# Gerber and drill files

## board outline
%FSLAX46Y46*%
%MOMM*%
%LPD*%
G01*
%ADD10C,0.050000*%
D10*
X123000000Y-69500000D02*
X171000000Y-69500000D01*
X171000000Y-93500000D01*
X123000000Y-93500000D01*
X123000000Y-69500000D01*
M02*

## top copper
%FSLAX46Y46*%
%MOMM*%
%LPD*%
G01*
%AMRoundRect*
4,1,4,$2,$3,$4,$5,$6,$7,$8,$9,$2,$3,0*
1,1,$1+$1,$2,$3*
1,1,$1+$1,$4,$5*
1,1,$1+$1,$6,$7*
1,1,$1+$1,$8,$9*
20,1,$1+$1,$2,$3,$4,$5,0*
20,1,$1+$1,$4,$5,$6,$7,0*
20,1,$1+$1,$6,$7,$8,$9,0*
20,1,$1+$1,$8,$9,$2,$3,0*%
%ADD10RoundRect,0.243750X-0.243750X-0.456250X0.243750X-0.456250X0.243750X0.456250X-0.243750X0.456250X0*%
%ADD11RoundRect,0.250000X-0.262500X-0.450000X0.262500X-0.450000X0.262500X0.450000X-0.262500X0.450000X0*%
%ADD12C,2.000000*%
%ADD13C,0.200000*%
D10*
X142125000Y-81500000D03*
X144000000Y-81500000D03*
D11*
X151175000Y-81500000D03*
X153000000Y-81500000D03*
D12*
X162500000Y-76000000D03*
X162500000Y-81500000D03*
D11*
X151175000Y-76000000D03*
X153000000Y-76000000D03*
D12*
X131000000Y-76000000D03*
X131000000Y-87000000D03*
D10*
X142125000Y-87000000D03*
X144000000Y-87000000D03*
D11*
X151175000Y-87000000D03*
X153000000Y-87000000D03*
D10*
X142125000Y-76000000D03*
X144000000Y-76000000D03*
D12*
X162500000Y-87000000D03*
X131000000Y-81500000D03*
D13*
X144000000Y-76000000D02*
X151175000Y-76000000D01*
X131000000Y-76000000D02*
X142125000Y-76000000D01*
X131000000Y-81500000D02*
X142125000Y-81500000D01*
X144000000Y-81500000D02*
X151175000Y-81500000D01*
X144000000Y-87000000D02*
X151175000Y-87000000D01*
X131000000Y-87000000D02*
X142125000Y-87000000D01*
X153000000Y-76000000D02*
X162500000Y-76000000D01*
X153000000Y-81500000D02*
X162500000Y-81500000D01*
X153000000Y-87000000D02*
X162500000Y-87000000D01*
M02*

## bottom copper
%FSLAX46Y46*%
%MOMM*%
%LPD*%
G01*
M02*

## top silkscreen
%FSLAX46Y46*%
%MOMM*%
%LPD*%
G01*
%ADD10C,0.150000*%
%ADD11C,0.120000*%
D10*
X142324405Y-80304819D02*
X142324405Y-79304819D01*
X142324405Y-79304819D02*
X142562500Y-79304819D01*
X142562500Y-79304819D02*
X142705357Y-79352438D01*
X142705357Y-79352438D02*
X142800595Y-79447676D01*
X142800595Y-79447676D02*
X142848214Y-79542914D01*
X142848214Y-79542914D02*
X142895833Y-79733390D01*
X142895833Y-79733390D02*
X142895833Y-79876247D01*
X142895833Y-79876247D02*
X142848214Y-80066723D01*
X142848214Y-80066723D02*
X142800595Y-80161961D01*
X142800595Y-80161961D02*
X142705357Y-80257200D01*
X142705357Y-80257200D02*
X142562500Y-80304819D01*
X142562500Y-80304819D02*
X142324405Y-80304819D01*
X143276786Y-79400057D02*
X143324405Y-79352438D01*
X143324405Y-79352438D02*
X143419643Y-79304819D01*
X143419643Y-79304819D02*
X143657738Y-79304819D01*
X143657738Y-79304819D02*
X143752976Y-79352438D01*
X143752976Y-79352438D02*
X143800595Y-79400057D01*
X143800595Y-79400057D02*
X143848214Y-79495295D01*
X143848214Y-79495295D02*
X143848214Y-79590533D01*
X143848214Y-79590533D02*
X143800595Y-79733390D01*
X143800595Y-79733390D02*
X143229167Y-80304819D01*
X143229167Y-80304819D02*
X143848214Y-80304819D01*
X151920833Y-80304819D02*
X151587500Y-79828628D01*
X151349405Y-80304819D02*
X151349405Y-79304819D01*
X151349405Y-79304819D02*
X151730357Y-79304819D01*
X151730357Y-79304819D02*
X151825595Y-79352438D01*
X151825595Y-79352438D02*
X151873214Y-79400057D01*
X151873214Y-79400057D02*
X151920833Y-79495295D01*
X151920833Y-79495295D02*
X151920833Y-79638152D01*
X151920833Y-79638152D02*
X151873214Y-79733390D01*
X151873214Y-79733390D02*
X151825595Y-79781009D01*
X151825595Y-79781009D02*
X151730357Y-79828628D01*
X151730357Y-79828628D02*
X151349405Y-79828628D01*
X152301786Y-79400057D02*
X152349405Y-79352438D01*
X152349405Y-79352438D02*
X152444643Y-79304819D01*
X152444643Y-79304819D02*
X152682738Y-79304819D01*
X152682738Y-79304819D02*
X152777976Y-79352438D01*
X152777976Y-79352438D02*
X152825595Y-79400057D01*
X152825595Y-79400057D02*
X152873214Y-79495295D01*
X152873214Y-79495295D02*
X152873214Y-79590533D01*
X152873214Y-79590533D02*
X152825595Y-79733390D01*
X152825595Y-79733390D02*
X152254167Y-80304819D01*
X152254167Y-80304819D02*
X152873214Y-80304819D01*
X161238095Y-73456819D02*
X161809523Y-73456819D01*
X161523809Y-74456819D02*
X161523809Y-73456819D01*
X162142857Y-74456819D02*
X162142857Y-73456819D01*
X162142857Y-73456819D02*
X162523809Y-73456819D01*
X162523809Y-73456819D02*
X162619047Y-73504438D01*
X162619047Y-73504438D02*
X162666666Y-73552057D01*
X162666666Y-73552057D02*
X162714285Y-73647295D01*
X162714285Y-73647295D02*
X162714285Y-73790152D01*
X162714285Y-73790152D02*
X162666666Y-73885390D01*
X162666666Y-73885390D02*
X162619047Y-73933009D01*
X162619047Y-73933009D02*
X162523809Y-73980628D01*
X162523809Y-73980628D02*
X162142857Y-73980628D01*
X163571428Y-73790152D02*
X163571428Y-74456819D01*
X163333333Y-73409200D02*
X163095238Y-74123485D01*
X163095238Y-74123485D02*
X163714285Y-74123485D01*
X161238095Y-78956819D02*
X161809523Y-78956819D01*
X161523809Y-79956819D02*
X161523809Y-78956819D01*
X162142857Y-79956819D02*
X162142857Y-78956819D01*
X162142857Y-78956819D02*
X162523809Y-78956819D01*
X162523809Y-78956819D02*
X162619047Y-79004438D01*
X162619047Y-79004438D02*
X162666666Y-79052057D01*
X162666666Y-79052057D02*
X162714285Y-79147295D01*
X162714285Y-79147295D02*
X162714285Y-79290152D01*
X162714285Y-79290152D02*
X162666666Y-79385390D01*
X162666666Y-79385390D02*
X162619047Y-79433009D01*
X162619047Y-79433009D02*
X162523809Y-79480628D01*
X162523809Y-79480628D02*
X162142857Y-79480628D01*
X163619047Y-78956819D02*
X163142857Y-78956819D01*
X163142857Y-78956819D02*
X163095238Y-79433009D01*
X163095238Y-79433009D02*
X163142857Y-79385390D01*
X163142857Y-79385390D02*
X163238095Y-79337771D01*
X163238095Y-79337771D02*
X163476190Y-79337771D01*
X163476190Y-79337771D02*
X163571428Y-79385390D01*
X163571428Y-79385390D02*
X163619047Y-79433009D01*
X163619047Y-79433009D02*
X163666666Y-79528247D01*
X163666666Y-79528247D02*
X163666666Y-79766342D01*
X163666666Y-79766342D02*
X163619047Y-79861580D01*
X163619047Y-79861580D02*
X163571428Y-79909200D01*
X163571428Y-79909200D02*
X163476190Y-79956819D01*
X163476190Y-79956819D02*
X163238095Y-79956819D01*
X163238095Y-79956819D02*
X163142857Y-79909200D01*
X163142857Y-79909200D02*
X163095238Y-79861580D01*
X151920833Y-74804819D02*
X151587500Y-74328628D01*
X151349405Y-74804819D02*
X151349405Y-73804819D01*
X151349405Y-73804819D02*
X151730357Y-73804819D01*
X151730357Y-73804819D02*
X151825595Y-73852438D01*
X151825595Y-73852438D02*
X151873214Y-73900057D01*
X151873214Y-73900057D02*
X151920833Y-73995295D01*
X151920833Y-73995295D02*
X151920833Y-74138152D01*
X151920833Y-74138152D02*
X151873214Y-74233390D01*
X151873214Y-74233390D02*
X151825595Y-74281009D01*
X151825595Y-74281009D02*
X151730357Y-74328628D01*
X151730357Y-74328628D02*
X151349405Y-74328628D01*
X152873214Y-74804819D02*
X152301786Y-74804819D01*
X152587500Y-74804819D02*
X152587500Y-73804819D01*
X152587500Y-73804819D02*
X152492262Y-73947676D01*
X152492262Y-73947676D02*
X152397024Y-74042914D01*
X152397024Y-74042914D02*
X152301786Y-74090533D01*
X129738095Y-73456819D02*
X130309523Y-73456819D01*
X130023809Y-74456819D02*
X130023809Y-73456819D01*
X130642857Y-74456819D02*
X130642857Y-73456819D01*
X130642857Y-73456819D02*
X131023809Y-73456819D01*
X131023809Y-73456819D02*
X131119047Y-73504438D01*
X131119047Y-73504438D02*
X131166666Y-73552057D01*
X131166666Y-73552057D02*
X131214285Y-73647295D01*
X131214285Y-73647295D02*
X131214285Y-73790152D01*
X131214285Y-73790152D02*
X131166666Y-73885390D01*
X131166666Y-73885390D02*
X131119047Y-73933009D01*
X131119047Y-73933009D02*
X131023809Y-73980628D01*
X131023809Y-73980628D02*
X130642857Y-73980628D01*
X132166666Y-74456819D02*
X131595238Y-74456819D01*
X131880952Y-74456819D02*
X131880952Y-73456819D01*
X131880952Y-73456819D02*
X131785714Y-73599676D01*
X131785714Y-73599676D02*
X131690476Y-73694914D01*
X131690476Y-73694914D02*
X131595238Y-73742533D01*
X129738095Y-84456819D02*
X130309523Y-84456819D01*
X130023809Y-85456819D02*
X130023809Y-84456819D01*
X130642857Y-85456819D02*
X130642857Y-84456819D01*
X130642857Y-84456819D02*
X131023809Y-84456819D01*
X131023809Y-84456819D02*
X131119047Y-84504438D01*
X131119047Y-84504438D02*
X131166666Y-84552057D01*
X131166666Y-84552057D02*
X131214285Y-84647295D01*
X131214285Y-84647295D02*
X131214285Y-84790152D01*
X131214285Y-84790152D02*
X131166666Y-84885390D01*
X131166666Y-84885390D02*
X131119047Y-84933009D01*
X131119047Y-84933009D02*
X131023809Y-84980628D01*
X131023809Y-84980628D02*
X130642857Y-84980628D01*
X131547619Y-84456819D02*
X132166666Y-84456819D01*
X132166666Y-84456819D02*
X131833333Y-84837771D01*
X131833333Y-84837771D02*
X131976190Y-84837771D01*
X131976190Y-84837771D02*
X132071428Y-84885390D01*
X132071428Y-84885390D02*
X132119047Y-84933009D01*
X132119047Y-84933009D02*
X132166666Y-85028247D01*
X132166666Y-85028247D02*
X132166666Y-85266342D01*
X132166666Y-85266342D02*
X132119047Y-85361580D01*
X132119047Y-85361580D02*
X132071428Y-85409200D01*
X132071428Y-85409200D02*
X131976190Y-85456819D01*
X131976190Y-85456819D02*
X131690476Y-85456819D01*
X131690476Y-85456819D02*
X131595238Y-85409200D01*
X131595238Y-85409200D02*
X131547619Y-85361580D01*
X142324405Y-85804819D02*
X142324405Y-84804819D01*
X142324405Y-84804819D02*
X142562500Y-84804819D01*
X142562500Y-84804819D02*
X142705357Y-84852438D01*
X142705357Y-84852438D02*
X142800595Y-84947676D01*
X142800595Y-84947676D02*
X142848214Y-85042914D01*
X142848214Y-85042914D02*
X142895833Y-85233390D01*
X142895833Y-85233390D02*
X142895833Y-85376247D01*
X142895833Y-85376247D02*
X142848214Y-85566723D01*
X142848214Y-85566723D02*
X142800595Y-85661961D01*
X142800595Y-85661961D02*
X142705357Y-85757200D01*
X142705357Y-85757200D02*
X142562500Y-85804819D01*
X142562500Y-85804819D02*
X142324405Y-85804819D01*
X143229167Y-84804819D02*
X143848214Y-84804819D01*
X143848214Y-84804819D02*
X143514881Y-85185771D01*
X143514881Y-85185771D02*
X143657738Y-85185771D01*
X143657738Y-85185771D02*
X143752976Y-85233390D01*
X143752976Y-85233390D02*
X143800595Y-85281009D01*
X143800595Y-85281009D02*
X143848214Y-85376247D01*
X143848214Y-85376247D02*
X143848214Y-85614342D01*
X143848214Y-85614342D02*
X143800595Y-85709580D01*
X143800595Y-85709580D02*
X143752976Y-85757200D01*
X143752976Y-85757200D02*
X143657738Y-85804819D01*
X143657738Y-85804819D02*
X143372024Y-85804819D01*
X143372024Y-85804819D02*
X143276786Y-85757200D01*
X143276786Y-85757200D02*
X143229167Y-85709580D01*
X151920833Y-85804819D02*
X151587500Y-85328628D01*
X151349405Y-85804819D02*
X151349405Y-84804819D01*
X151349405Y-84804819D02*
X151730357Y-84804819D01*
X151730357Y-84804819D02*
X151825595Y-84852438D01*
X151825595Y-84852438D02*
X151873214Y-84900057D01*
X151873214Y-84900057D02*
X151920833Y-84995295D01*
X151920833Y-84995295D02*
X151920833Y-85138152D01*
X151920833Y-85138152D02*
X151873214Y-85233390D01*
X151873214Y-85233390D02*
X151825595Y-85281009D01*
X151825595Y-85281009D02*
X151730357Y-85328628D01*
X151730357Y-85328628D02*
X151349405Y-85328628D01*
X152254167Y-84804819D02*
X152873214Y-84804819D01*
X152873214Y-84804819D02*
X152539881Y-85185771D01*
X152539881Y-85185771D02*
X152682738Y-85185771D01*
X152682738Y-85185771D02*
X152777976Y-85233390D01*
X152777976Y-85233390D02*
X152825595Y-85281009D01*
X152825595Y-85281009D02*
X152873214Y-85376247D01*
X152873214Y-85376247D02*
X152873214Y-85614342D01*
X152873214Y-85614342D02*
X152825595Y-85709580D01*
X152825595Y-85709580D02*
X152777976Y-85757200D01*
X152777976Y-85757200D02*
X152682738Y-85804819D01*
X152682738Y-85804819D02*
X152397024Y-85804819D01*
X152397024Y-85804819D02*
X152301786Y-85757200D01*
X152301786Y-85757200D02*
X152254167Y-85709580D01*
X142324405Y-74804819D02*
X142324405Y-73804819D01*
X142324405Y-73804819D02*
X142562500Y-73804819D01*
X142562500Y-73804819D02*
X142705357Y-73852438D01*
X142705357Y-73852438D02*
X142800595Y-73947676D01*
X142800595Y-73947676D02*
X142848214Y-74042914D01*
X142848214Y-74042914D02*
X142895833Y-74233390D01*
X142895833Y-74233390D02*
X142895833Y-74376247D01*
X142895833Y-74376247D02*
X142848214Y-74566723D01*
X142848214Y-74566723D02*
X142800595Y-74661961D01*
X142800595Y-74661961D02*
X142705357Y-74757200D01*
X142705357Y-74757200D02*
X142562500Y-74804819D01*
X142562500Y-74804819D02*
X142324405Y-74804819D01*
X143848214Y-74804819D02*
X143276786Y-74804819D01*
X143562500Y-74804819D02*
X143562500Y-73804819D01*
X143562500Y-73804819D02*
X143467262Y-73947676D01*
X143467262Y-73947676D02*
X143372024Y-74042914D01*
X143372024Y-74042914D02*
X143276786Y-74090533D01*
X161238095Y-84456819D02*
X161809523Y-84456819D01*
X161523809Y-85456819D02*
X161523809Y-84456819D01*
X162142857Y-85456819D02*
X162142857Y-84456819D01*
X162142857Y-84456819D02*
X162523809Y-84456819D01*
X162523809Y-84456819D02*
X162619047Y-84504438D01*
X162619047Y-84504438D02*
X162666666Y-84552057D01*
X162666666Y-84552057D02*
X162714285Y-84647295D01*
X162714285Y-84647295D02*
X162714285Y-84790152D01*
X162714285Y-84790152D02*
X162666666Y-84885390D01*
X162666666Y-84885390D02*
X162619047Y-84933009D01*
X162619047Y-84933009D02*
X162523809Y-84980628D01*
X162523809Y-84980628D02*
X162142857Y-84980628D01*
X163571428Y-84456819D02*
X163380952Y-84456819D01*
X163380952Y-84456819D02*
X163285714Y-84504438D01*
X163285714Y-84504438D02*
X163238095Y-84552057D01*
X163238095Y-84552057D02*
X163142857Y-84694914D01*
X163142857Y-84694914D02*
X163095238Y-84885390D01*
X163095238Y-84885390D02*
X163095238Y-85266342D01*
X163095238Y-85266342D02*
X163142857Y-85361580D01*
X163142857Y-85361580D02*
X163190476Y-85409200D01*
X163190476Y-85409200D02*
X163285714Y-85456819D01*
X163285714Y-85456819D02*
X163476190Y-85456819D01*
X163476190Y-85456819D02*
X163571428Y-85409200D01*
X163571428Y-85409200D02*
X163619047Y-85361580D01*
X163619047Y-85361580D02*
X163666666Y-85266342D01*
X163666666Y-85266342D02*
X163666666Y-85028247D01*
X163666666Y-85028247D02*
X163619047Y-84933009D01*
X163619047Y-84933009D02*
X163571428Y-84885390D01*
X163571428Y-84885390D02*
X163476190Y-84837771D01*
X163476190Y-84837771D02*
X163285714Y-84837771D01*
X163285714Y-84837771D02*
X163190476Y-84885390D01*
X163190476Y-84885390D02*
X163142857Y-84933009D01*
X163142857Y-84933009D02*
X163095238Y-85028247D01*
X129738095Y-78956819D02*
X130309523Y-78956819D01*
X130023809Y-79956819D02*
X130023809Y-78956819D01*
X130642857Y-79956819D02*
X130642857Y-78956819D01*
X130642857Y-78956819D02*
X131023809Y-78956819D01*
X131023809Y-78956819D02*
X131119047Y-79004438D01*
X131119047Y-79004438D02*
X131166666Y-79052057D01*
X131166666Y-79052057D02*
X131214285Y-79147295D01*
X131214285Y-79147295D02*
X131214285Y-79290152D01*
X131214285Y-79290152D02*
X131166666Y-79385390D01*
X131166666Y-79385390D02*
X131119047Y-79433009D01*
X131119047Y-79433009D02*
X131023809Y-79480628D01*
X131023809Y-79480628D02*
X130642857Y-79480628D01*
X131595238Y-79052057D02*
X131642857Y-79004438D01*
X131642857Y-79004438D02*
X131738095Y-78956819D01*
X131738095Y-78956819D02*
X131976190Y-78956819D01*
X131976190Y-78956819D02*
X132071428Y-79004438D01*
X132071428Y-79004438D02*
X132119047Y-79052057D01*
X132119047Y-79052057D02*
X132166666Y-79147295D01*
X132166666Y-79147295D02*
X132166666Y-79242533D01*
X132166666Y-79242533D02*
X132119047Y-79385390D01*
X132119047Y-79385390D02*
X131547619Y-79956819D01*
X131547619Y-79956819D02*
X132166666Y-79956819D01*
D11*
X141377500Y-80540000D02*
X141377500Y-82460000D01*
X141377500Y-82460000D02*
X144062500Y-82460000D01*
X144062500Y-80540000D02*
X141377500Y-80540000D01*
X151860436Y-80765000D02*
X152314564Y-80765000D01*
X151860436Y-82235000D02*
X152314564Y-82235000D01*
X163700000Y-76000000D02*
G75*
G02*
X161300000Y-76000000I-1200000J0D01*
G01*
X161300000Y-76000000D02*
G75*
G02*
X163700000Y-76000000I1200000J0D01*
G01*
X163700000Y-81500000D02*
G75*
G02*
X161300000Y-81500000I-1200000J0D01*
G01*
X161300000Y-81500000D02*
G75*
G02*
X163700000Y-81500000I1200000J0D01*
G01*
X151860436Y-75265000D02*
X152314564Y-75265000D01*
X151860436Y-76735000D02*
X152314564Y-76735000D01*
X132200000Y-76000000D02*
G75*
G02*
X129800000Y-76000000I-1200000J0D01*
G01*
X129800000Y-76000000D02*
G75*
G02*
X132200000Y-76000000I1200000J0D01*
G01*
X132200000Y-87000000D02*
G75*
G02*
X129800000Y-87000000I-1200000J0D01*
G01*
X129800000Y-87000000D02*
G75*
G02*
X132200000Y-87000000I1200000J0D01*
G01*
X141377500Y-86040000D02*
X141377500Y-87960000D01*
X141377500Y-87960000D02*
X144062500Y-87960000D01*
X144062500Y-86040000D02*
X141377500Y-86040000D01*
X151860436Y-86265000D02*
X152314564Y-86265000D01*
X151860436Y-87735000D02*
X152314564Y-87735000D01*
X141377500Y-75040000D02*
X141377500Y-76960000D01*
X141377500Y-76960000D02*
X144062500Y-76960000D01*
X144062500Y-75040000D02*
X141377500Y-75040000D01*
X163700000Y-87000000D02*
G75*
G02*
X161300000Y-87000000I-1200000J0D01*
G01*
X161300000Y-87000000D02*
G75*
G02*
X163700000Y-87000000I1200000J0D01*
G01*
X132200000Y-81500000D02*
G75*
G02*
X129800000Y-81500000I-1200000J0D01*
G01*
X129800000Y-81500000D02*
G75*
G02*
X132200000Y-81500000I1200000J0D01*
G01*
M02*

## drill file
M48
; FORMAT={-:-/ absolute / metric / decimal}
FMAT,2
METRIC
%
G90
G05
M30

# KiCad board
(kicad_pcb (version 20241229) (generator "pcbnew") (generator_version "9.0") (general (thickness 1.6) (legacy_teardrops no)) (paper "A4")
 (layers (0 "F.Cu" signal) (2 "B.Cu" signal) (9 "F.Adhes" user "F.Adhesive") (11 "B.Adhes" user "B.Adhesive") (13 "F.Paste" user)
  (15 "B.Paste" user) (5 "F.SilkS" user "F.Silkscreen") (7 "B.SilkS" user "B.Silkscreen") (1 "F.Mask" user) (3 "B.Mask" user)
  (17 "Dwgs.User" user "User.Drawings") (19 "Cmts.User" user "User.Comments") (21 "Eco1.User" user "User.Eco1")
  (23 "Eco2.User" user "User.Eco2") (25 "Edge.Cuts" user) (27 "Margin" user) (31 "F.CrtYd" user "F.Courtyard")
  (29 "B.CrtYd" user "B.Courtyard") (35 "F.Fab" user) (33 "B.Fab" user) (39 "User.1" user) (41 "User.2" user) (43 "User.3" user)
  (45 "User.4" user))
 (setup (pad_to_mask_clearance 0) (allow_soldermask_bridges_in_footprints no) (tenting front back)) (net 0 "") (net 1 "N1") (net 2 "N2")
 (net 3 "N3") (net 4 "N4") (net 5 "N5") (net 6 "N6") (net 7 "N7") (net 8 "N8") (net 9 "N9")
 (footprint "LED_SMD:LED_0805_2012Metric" (layer "F.Cu") (at 143.0625 81.5)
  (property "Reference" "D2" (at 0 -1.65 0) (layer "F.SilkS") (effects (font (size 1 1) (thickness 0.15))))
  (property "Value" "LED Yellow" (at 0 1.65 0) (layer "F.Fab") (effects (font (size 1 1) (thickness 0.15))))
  (fp_line (start -1.685 -0.96) (end -1.685 0.96) (stroke (width 0.12) (type solid)) (layer "F.SilkS"))
  (fp_line (start -1.685 0.96) (end 1 0.96) (stroke (width 0.12) (type solid)) (layer "F.SilkS"))
  (fp_line (start 1 -0.96) (end -1.685 -0.96) (stroke (width 0.12) (type solid)) (layer "F.SilkS"))
  (pad "1" smd roundrect (at -0.9375 0) (size 0.975 1.4) (layers "F.Cu" "F.Mask" "F.Paste") (roundrect_rratio 0.25) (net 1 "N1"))
  (pad "2" smd roundrect (at 0.9375 0) (size 0.975 1.4) (layers "F.Cu" "F.Mask" "F.Paste") (roundrect_rratio 0.25) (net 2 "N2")))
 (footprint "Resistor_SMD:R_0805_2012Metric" (layer "F.Cu") (at 152.0875 81.5)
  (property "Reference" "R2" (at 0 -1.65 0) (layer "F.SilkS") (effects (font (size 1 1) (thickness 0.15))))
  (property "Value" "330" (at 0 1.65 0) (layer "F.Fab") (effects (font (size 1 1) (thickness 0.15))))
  (fp_line (start -0.227064 -0.735) (end 0.227064 -0.735) (stroke (width 0.12) (type solid)) (layer "F.SilkS"))
  (fp_line (start -0.227064 0.735) (end 0.227064 0.735) (stroke (width 0.12) (type solid)) (layer "F.SilkS"))
  (pad "1" smd roundrect (at -0.9125 0) (size 1.025 1.4) (layers "F.Cu" "F.Mask" "F.Paste") (roundrect_rratio 0.243902) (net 2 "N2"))
  (pad "2" smd roundrect (at 0.9125 0) (size 1.025 1.4) (layers "F.Cu" "F.Mask" "F.Paste") (roundrect_rratio 0.243902) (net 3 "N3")))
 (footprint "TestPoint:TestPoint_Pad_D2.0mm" (layer "F.Cu") (at 162.5 76)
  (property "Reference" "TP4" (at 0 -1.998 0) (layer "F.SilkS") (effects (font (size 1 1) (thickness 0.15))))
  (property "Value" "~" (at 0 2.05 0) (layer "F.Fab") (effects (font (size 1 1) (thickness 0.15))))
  (fp_circle (center 0 0) (end 0 1.2) (stroke (width 0.12) (type solid)) (fill no) (layer "F.SilkS"))
  (pad "1" smd circle (at 0 0) (size 2 2) (layers "F.Cu" "F.Mask") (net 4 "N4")))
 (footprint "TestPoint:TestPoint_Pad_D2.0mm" (layer "F.Cu") (at 162.5 81.5)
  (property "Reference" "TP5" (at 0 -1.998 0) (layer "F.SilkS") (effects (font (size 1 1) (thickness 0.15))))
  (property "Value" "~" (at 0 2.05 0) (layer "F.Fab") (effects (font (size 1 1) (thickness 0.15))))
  (fp_circle (center 0 0) (end 0 1.2) (stroke (width 0.12) (type solid)) (fill no) (layer "F.SilkS"))
  (pad "1" smd circle (at 0 0) (size 2 2) (layers "F.Cu" "F.Mask") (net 3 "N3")))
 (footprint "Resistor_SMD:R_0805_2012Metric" (layer "F.Cu") (at 152.0875 76)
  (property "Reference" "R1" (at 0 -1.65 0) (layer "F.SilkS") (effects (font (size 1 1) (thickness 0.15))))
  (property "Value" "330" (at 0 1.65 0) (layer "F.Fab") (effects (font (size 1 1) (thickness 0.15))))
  (fp_line (start -0.227064 -0.735) (end 0.227064 -0.735) (stroke (width 0.12) (type solid)) (layer "F.SilkS"))
  (fp_line (start -0.227064 0.735) (end 0.227064 0.735) (stroke (width 0.12) (type solid)) (layer "F.SilkS"))
  (pad "1" smd roundrect (at -0.9125 0) (size 1.025 1.4) (layers "F.Cu" "F.Mask" "F.Paste") (roundrect_rratio 0.243902) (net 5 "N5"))
  (pad "2" smd roundrect (at 0.9125 0) (size 1.025 1.4) (layers "F.Cu" "F.Mask" "F.Paste") (roundrect_rratio 0.243902) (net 4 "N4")))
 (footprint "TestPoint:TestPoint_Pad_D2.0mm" (layer "F.Cu") (at 131 76)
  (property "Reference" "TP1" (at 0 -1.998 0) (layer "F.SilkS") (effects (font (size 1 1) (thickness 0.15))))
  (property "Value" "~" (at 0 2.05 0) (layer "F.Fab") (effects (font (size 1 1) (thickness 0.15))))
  (fp_circle (center 0 0) (end 0 1.2) (stroke (width 0.12) (type solid)) (fill no) (layer "F.SilkS"))
  (pad "1" smd circle (at 0 0) (size 2 2) (layers "F.Cu" "F.Mask") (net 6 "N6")))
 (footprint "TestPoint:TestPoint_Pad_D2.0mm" (layer "F.Cu") (at 131 87)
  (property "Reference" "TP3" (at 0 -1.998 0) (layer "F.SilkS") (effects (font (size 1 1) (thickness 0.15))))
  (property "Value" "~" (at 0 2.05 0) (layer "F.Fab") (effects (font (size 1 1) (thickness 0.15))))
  (fp_circle (center 0 0) (end 0 1.2) (stroke (width 0.12) (type solid)) (fill no) (layer "F.SilkS"))
  (pad "1" smd circle (at 0 0) (size 2 2) (layers "F.Cu" "F.Mask") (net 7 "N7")))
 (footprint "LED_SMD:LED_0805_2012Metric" (layer "F.Cu") (at 143.0625 87)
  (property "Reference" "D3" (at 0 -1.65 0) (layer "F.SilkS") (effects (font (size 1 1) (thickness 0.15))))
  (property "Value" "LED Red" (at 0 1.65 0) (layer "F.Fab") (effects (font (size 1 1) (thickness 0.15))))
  (fp_line (start -1.685 -0.96) (end -1.685 0.96) (stroke (width 0.12) (type solid)) (layer "F.SilkS"))
  (fp_line (start -1.685 0.96) (end 1 0.96) (stroke (width 0.12) (type solid)) (layer "F.SilkS"))
  (fp_line (start 1 -0.96) (end -1.685 -0.96) (stroke (width 0.12) (type solid)) (layer "F.SilkS"))
  (pad "1" smd roundrect (at -0.9375 0) (size 0.975 1.4) (layers "F.Cu" "F.Mask" "F.Paste") (roundrect_rratio 0.25) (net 7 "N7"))
  (pad "2" smd roundrect (at 0.9375 0) (size 0.975 1.4) (layers "F.Cu" "F.Mask" "F.Paste") (roundrect_rratio 0.25) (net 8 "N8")))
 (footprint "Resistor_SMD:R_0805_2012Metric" (layer "F.Cu") (at 152.0875 87)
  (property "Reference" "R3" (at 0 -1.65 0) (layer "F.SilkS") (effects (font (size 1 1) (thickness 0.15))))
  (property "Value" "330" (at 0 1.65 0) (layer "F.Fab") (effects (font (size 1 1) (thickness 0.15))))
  (fp_line (start -0.227064 -0.735) (end 0.227064 -0.735) (stroke (width 0.12) (type solid)) (layer "F.SilkS"))
  (fp_line (start -0.227064 0.735) (end 0.227064 0.735) (stroke (width 0.12) (type solid)) (layer "F.SilkS"))
  (pad "1" smd roundrect (at -0.9125 0) (size 1.025 1.4) (layers "F.Cu" "F.Mask" "F.Paste") (roundrect_rratio 0.243902) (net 8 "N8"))
  (pad "2" smd roundrect (at 0.9125 0) (size 1.025 1.4) (layers "F.Cu" "F.Mask" "F.Paste") (roundrect_rratio 0.243902) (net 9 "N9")))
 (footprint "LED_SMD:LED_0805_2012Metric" (layer "F.Cu") (at 143.0625 76)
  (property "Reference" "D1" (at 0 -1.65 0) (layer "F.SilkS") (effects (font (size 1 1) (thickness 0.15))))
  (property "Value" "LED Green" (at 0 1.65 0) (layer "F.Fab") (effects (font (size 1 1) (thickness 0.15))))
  (fp_line (start -1.685 -0.96) (end -1.685 0.96) (stroke (width 0.12) (type solid)) (layer "F.SilkS"))
  (fp_line (start -1.685 0.96) (end 1 0.96) (stroke (width 0.12) (type solid)) (layer "F.SilkS"))
  (fp_line (start 1 -0.96) (end -1.685 -0.96) (stroke (width 0.12) (type solid)) (layer "F.SilkS"))
  (pad "1" smd roundrect (at -0.9375 0) (size 0.975 1.4) (layers "F.Cu" "F.Mask" "F.Paste") (roundrect_rratio 0.25) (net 6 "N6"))
  (pad "2" smd roundrect (at 0.9375 0) (size 0.975 1.4) (layers "F.Cu" "F.Mask" "F.Paste") (roundrect_rratio 0.25) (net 5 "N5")))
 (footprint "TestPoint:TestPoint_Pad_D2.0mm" (layer "F.Cu") (at 162.5 87)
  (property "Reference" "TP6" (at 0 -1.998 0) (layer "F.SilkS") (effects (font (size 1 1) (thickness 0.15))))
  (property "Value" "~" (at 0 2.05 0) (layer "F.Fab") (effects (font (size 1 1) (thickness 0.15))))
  (fp_circle (center 0 0) (end 0 1.2) (stroke (width 0.12) (type solid)) (fill no) (layer "F.SilkS"))
  (pad "1" smd circle (at 0 0) (size 2 2) (layers "F.Cu" "F.Mask") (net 9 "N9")))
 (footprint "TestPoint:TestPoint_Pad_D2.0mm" (layer "F.Cu") (at 131 81.5)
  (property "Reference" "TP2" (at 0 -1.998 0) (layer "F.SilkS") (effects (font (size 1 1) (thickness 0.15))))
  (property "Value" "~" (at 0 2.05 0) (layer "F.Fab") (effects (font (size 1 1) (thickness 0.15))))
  (fp_circle (center 0 0) (end 0 1.2) (stroke (width 0.12) (type solid)) (fill no) (layer "F.SilkS"))
  (pad "1" smd circle (at 0 0) (size 2 2) (layers "F.Cu" "F.Mask") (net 1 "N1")))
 (gr_rect (start 123 69.5) (end 171 93.5) (stroke (width 0.05) (type default)) (fill no) (layer "Edge.Cuts"))
 (segment (start 144 76) (end 151.175 76) (width 0.2) (layer "F.Cu") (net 5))
 (segment (start 131 76) (end 142.125 76) (width 0.2) (layer "F.Cu") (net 6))
 (segment (start 131 81.5) (end 142.125 81.5) (width 0.2) (layer "F.Cu") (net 1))
 (segment (start 144 81.5) (end 151.175 81.5) (width 0.2) (layer "F.Cu") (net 2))
 (segment (start 144 87) (end 151.175 87) (width 0.2) (layer "F.Cu") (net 8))
 (segment (start 131 87) (end 142.125 87) (width 0.2) (layer "F.Cu") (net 7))
 (segment (start 153 76) (end 162.5 76) (width 0.2) (layer "F.Cu") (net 4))
 (segment (start 153 81.5) (end 162.5 81.5) (width 0.2) (layer "F.Cu") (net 3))
 (segment (start 153 87) (end 162.5 87) (width 0.2) (layer "F.Cu") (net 9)))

